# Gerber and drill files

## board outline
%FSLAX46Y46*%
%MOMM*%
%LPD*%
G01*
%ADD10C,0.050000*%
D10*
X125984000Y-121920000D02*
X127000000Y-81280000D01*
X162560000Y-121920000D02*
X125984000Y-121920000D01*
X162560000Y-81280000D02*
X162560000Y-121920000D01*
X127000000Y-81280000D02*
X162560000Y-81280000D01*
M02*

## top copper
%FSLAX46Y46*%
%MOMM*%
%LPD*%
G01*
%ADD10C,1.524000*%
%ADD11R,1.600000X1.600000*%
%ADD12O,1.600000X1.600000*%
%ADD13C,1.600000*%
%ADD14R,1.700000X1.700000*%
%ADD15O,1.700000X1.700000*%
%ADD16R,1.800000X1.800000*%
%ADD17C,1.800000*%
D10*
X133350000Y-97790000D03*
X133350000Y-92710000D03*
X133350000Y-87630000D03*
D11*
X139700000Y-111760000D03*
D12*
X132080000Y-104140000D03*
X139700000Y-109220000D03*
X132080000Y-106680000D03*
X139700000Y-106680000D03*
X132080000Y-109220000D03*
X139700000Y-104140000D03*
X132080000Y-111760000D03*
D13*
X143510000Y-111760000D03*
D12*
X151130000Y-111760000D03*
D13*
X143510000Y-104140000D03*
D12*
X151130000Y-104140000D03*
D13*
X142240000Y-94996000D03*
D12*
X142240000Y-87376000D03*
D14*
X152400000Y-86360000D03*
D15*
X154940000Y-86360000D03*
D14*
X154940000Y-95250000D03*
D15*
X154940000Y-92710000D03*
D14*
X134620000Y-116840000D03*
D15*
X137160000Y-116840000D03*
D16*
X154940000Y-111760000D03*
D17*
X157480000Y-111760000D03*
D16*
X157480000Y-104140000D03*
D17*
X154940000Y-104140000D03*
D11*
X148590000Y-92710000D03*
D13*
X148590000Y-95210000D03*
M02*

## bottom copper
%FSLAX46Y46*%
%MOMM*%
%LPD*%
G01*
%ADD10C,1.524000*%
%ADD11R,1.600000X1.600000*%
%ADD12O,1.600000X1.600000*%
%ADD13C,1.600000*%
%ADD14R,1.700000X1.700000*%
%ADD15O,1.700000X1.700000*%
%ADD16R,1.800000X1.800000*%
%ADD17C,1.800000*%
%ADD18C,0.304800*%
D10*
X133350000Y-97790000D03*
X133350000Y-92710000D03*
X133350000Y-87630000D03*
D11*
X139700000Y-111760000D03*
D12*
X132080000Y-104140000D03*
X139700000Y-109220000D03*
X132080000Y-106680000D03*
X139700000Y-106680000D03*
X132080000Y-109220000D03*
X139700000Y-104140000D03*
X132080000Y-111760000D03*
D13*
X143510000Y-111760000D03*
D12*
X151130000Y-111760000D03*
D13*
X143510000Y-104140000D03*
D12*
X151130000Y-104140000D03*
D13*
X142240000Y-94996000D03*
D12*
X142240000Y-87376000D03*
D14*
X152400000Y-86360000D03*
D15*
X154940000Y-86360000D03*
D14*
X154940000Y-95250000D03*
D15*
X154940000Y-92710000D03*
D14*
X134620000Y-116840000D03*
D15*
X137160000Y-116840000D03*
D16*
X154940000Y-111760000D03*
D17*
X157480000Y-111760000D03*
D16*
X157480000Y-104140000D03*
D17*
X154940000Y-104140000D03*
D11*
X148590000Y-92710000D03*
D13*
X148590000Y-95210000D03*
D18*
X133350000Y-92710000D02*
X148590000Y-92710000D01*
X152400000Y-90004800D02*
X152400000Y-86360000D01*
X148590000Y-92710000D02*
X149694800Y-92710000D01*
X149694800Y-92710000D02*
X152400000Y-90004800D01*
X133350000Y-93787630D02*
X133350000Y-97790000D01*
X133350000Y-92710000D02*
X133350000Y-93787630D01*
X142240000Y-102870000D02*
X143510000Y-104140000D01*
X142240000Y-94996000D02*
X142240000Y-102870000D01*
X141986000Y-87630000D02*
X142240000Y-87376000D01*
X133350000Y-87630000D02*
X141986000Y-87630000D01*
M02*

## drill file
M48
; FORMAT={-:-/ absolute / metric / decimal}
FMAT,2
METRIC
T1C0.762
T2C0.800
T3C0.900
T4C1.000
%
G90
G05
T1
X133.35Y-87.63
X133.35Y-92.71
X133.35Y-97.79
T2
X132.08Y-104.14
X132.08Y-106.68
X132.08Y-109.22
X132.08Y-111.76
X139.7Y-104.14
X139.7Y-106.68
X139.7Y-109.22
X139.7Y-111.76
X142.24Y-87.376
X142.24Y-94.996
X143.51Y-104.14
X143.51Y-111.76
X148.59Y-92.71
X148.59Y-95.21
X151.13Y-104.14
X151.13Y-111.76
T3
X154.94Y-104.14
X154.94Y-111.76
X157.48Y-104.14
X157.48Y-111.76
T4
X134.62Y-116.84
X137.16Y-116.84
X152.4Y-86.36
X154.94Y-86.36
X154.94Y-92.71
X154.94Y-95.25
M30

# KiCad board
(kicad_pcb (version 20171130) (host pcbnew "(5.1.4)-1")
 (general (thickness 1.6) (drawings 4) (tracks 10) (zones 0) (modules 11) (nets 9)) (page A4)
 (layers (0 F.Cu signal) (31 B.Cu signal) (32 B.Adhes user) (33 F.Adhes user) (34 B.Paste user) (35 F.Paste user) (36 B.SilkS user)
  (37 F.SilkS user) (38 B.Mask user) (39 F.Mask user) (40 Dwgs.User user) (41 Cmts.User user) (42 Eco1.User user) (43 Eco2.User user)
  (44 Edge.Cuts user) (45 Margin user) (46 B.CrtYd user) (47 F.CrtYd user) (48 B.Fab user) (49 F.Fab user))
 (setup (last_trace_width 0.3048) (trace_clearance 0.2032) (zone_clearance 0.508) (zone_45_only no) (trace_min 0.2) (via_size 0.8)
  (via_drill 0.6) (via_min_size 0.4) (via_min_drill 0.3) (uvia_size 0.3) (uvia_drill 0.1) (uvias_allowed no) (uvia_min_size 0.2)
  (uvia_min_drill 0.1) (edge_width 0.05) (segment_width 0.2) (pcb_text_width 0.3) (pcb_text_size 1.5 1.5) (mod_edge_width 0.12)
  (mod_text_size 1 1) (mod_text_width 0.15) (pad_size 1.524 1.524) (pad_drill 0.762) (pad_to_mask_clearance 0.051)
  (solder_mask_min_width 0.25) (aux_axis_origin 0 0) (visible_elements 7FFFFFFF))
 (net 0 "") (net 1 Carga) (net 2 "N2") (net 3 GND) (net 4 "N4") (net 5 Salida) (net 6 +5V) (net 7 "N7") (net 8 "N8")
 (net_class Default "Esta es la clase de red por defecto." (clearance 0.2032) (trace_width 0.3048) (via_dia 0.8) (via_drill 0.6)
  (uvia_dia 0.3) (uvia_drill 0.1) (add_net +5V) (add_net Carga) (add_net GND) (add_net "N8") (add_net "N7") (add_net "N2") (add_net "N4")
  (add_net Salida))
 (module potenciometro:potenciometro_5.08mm (layer F.Cu) (at 133.35 102.87)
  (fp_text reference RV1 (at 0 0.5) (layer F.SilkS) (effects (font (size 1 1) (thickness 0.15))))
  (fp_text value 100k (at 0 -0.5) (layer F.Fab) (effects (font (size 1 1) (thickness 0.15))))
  (pad 3 thru_hole circle (at 0 -5.08) (size 1.524 1.524) (drill 0.762) (layers *.Cu *.Mask) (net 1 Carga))
  (pad 2 thru_hole circle (at 0 -10.16) (size 1.524 1.524) (drill 0.762) (layers *.Cu *.Mask) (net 1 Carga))
  (pad 1 thru_hole circle (at 0 -15.24) (size 1.524 1.524) (drill 0.762) (layers *.Cu *.Mask) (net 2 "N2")))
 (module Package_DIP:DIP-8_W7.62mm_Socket (layer F.Cu) (at 139.7 111.76 180)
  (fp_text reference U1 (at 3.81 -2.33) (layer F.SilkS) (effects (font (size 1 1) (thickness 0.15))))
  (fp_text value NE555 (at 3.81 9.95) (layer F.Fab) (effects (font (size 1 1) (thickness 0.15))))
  (pad 1 thru_hole rect (at 0 0 180) (size 1.6 1.6) (drill 0.8) (layers *.Cu *.Mask) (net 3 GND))
  (pad 5 thru_hole oval (at 7.62 7.62 180) (size 1.6 1.6) (drill 0.8) (layers *.Cu *.Mask) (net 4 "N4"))
  (pad 2 thru_hole oval (at 0 2.54 180) (size 1.6 1.6) (drill 0.8) (layers *.Cu *.Mask) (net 1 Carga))
  (pad 6 thru_hole oval (at 7.62 5.08 180) (size 1.6 1.6) (drill 0.8) (layers *.Cu *.Mask) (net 1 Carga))
  (pad 3 thru_hole oval (at 0 5.08 180) (size 1.6 1.6) (drill 0.8) (layers *.Cu *.Mask) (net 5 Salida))
  (pad 7 thru_hole oval (at 7.62 2.54 180) (size 1.6 1.6) (drill 0.8) (layers *.Cu *.Mask) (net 2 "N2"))
  (pad 4 thru_hole oval (at 0 7.62 180) (size 1.6 1.6) (drill 0.8) (layers *.Cu *.Mask) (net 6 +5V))
  (pad 8 thru_hole oval (at 7.62 0 180) (size 1.6 1.6) (drill 0.8) (layers *.Cu *.Mask) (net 6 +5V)))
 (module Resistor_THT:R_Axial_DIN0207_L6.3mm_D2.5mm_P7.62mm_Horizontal (layer F.Cu) (at 143.51 111.76)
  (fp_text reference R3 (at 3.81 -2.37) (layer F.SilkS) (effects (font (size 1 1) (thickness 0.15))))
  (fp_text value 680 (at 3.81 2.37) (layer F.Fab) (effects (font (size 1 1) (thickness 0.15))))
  (pad 1 thru_hole circle (at 0 0) (size 1.6 1.6) (drill 0.8) (layers *.Cu *.Mask) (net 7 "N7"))
  (pad 2 thru_hole oval (at 7.62 0) (size 1.6 1.6) (drill 0.8) (layers *.Cu *.Mask) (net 3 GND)))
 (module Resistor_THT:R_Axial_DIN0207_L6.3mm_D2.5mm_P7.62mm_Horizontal (layer F.Cu) (at 143.51 104.14)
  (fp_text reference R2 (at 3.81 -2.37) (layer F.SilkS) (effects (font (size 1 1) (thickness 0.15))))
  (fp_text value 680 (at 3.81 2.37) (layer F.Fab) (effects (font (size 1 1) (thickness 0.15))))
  (pad 1 thru_hole circle (at 0 0) (size 1.6 1.6) (drill 0.8) (layers *.Cu *.Mask) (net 6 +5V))
  (pad 2 thru_hole oval (at 7.62 0) (size 1.6 1.6) (drill 0.8) (layers *.Cu *.Mask) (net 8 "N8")))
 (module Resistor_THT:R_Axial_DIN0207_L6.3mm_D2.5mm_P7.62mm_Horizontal (layer F.Cu) (at 142.24 94.996 90)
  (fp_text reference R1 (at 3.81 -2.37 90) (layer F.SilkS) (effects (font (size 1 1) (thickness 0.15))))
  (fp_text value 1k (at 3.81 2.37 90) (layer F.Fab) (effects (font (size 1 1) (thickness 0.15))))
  (pad 1 thru_hole circle (at 0 0 90) (size 1.6 1.6) (drill 0.8) (layers *.Cu *.Mask) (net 6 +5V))
  (pad 2 thru_hole oval (at 7.62 0 90) (size 1.6 1.6) (drill 0.8) (layers *.Cu *.Mask) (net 2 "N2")))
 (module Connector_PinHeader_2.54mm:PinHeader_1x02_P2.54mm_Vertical (layer F.Cu) (at 152.4 86.36 90)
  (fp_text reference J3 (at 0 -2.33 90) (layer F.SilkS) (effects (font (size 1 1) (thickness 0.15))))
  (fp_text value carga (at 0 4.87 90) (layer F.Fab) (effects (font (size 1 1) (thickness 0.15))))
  (pad 1 thru_hole rect (at 0 0 90) (size 1.7 1.7) (drill 1) (layers *.Cu *.Mask) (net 1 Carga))
  (pad 2 thru_hole oval (at 0 2.54 90) (size 1.7 1.7) (drill 1) (layers *.Cu *.Mask) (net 3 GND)))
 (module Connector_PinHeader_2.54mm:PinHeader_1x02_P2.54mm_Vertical (layer F.Cu) (at 154.94 95.25 180)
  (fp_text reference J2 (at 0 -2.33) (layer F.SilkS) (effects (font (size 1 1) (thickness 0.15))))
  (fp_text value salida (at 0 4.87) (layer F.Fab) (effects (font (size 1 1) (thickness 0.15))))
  (pad 1 thru_hole rect (at 0 0 180) (size 1.7 1.7) (drill 1) (layers *.Cu *.Mask) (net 5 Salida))
  (pad 2 thru_hole oval (at 0 2.54 180) (size 1.7 1.7) (drill 1) (layers *.Cu *.Mask) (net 3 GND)))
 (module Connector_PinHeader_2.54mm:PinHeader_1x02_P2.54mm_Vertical (layer F.Cu) (at 134.62 116.84 90)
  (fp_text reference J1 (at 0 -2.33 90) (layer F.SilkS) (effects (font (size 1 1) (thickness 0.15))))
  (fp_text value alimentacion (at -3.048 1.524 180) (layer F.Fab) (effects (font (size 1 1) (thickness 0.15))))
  (pad 1 thru_hole rect (at 0 0 90) (size 1.7 1.7) (drill 1) (layers *.Cu *.Mask) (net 6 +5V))
  (pad 2 thru_hole oval (at 0 2.54 90) (size 1.7 1.7) (drill 1) (layers *.Cu *.Mask) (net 3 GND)))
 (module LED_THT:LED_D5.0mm (layer F.Cu) (at 154.94 111.76)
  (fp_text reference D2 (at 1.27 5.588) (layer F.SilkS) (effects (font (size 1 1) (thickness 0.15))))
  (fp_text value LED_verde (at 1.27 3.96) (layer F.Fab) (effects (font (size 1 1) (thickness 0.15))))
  (pad 1 thru_hole rect (at 0 0) (size 1.8 1.8) (drill 0.9) (layers *.Cu *.Mask) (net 7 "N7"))
  (pad 2 thru_hole circle (at 2.54 0) (size 1.8 1.8) (drill 0.9) (layers *.Cu *.Mask) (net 5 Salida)))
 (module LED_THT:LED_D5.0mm (layer F.Cu) (at 157.48 104.14 180)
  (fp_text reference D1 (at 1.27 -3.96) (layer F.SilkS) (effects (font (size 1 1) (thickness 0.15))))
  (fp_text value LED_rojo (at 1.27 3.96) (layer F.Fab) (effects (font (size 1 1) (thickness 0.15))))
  (pad 1 thru_hole rect (at 0 0 180) (size 1.8 1.8) (drill 0.9) (layers *.Cu *.Mask) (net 5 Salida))
  (pad 2 thru_hole circle (at 2.54 0 180) (size 1.8 1.8) (drill 0.9) (layers *.Cu *.Mask) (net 8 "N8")))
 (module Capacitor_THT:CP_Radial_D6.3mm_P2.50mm (layer F.Cu) (at 148.59 92.71 270)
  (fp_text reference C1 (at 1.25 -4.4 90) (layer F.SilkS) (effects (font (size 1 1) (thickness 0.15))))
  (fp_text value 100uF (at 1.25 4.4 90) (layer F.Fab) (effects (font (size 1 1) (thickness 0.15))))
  (pad 1 thru_hole rect (at 0 0 270) (size 1.6 1.6) (drill 0.8) (layers *.Cu *.Mask) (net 1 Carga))
  (pad 2 thru_hole circle (at 2.5 0 270) (size 1.6 1.6) (drill 0.8) (layers *.Cu *.Mask) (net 3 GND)))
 (gr_line (start 125.984 121.92) (end 127 81.28) (layer Edge.Cuts) (width 0.05))
 (gr_line (start 162.56 121.92) (end 125.984 121.92) (layer Edge.Cuts) (width 0.05))
 (gr_line (start 162.56 81.28) (end 162.56 121.92) (layer Edge.Cuts) (width 0.05))
 (gr_line (start 127 81.28) (end 162.56 81.28) (layer Edge.Cuts) (width 0.05))
 (segment (start 133.35 92.71) (end 148.59 92.71) (width 0.3048) (layer B.Cu) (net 1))
 (segment (start 152.4 90.0048) (end 152.4 86.36) (width 0.3048) (layer B.Cu) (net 1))
 (segment (start 148.59 92.71) (end 149.6948 92.71) (width 0.3048) (layer B.Cu) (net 1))
 (segment (start 149.6948 92.71) (end 152.4 90.0048) (width 0.3048) (layer B.Cu) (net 1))
 (segment (start 133.35 93.78763) (end 133.35 97.79) (width 0.3048) (layer B.Cu) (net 1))
 (segment (start 133.35 92.71) (end 133.35 93.78763) (width 0.3048) (layer B.Cu) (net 1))
 (segment (start 142.24 102.87) (end 143.51 104.14) (width 0.3048) (layer B.Cu) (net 6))
 (segment (start 142.24 94.996) (end 142.24 102.87) (width 0.3048) (layer B.Cu) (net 6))
 (segment (start 141.986 87.63) (end 142.24 87.376) (width 0.3048) (layer B.Cu) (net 2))
 (segment (start 133.35 87.63) (end 141.986 87.63) (width 0.3048) (layer B.Cu) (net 2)))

